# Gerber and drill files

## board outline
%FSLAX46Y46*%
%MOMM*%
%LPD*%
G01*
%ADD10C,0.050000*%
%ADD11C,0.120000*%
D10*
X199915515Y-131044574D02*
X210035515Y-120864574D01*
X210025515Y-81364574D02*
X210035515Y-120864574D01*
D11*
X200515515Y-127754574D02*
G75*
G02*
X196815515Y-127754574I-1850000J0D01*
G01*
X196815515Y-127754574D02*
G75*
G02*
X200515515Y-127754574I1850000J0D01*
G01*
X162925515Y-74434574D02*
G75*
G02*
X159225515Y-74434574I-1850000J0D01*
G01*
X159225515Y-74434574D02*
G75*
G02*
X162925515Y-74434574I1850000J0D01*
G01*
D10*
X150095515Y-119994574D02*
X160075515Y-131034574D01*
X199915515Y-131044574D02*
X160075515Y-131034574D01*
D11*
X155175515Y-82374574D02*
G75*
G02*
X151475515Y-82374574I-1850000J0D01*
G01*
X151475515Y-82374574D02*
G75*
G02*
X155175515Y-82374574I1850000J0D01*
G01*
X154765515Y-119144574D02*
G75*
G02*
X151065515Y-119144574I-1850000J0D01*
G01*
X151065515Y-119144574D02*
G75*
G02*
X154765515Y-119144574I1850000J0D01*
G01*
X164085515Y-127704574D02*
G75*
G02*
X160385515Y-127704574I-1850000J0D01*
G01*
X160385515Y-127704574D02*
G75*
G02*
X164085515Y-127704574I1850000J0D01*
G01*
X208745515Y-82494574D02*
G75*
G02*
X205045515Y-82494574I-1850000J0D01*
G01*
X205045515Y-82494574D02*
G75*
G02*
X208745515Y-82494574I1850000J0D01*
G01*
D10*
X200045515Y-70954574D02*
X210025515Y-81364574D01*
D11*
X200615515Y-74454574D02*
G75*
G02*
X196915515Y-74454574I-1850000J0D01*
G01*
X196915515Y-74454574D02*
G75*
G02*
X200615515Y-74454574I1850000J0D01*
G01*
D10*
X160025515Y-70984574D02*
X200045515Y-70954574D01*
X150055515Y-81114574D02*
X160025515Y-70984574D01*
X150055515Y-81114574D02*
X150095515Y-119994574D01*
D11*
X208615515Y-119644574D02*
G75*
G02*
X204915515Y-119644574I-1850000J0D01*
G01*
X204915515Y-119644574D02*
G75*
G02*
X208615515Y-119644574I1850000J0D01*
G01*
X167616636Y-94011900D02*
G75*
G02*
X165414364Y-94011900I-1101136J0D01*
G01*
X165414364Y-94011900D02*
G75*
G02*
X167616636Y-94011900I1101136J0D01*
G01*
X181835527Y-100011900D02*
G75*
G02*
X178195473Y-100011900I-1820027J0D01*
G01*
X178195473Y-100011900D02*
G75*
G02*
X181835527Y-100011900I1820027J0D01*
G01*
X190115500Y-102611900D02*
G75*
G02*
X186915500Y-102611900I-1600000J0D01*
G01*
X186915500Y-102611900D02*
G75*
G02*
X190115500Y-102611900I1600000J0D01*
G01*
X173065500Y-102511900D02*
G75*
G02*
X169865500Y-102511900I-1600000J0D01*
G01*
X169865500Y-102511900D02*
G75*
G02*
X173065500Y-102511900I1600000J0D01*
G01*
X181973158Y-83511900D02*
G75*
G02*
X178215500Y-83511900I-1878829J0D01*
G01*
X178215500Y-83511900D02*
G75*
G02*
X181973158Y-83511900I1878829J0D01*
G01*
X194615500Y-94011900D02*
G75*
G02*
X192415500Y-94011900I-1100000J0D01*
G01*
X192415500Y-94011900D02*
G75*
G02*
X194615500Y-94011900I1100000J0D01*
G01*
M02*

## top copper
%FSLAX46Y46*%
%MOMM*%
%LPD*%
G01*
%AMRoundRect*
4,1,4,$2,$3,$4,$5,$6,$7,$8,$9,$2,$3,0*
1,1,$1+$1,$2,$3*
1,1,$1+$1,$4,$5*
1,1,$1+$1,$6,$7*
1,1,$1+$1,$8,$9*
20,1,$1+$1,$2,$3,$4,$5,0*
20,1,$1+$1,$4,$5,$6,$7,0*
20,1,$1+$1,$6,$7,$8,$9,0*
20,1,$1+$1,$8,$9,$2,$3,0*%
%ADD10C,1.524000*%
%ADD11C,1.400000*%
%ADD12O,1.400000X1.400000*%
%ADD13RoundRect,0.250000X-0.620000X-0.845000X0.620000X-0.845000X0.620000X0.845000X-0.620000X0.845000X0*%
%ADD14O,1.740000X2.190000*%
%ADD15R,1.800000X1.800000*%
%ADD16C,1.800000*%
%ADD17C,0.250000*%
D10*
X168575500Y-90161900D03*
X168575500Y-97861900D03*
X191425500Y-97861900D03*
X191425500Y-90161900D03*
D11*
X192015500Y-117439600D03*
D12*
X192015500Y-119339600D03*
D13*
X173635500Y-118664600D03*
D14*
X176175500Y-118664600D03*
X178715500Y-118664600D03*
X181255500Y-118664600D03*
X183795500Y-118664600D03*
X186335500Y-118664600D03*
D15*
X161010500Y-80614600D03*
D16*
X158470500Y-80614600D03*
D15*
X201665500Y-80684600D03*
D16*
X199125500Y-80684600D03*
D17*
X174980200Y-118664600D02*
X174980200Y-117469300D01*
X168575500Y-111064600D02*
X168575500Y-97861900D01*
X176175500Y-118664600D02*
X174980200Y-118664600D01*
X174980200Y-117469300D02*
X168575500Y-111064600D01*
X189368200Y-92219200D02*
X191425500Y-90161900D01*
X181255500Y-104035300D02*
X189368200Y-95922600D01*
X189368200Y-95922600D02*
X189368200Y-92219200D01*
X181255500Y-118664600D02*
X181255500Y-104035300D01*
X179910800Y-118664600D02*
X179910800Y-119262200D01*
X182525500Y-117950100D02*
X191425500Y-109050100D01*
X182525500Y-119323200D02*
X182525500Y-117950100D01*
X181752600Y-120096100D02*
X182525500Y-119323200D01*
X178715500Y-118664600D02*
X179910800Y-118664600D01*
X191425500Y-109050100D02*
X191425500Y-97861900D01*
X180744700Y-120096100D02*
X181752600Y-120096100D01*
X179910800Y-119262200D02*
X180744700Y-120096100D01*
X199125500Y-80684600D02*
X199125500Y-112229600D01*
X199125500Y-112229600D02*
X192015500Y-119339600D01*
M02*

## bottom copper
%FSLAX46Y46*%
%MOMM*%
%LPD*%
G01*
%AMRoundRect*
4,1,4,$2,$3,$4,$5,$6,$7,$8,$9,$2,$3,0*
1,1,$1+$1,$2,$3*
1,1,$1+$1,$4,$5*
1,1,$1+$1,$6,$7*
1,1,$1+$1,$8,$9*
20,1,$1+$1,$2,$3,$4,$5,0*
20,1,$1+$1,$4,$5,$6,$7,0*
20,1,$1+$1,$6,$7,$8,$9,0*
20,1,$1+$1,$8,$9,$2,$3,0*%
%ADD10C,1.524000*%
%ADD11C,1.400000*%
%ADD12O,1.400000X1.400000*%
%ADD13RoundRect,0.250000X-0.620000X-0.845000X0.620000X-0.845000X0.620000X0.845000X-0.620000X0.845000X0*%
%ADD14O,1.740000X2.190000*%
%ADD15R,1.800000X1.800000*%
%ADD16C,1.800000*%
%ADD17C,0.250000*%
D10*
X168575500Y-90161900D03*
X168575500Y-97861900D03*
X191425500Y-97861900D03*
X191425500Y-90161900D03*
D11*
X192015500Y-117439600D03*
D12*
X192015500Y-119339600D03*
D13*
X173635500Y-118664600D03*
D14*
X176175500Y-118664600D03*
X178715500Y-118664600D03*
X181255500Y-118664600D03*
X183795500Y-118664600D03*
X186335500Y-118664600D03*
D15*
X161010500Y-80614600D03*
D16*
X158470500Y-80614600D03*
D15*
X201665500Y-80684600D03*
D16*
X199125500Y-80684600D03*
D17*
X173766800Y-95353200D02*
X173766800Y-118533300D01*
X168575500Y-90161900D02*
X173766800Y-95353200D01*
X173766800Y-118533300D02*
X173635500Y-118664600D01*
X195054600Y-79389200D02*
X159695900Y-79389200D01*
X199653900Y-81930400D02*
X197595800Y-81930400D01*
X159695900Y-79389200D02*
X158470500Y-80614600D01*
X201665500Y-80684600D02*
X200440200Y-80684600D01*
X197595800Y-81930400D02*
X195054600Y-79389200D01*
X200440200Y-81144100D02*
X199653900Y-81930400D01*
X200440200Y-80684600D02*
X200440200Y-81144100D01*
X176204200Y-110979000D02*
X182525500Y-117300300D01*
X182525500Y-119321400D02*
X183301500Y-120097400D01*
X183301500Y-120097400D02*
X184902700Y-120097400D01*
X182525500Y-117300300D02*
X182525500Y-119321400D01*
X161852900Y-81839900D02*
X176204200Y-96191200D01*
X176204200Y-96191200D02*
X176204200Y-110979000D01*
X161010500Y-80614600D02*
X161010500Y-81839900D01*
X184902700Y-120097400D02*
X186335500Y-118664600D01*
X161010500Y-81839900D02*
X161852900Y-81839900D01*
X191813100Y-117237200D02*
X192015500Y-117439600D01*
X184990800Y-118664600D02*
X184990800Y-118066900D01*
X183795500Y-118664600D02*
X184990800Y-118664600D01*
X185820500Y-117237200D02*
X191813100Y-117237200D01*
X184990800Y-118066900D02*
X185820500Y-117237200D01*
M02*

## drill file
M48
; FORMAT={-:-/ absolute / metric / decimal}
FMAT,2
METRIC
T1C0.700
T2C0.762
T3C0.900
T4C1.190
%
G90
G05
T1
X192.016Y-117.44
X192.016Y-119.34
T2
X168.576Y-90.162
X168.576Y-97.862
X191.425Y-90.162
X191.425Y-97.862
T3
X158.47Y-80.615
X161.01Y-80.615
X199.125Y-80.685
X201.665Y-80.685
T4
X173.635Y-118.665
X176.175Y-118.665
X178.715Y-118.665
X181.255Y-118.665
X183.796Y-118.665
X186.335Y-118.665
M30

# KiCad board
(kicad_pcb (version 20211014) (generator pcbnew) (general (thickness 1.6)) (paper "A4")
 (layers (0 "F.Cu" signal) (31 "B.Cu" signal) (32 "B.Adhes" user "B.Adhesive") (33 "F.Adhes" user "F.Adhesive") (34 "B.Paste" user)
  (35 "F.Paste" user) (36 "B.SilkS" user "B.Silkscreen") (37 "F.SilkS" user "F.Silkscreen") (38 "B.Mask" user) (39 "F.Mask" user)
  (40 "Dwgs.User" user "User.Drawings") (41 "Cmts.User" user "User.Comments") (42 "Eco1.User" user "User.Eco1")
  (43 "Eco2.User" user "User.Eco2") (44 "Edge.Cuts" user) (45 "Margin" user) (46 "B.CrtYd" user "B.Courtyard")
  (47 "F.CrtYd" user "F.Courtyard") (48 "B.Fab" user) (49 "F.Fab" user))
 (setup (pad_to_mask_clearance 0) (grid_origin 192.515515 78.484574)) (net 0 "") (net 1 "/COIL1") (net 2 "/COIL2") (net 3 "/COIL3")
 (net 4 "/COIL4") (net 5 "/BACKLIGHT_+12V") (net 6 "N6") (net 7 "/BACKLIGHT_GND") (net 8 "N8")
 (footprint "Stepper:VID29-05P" (layer "F.Cu") (at 180.0155 94.0119)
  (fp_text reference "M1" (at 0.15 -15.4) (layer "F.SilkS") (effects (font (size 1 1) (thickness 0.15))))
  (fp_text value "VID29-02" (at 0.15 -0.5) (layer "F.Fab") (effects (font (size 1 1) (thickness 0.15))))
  (fp_circle (center -13.5 0) (end -12.65 0.7) (layer "Edge.Cuts") (width 0.12) (fill none))
  (fp_circle (center 0 6) (end 1.45 7.1) (layer "Edge.Cuts") (width 0.12) (fill none))
  (fp_circle (center 8.5 8.6) (end 10.1 8.6) (layer "Edge.Cuts") (width 0.12) (fill none))
  (fp_circle (center -8.55 8.5) (end -6.95 8.5) (layer "Edge.Cuts") (width 0.12) (fill none))
  (fp_circle (center 0.078829 -10.5) (end 1.778829 -9.7) (layer "Edge.Cuts") (width 0.12) (fill none))
  (fp_circle (center 13.5 0) (end 14.6 0) (layer "Edge.Cuts") (width 0.12) (fill none))
  (pad "1" thru_hole circle (at -11.44 -3.85) (size 1.524 1.524) (drill 0.762) (layers *.Cu *.Mask) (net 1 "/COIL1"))
  (pad "2" thru_hole circle (at -11.44 3.85) (size 1.524 1.524) (drill 0.762) (layers *.Cu *.Mask) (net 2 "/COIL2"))
  (pad "3" thru_hole circle (at 11.41 3.85) (size 1.524 1.524) (drill 0.762) (layers *.Cu *.Mask) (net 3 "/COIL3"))
  (pad "4" thru_hole circle (at 11.41 -3.85) (size 1.524 1.524) (drill 0.762) (layers *.Cu *.Mask) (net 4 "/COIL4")))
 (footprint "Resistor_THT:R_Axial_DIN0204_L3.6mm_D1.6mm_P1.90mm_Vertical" (layer "F.Cu") (at 192.0155 117.4396 -90)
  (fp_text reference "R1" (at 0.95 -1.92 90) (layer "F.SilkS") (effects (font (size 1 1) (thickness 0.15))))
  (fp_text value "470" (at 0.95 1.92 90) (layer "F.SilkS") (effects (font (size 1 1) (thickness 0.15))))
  (pad "1" thru_hole circle (at 0 0 270) (size 1.4 1.4) (drill 0.7) (layers *.Cu *.Mask) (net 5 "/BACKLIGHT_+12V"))
  (pad "2" thru_hole oval (at 1.9 0 270) (size 1.4 1.4) (drill 0.7) (layers *.Cu *.Mask) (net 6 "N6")))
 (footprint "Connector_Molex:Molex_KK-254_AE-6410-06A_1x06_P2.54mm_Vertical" (layer "F.Cu") (at 173.6355 118.6646)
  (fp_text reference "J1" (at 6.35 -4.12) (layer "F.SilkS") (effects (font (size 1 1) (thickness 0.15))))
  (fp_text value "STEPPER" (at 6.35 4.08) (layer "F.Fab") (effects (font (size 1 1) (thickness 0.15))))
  (pad "1" thru_hole roundrect (at 0 0) (size 1.74 2.19) (drill 1.19) (layers *.Cu *.Mask) (roundrect_rratio 0.1436781609) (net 1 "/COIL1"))
  (pad "2" thru_hole oval (at 2.54 0) (size 1.74 2.19) (drill 1.19) (layers *.Cu *.Mask) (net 2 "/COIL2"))
  (pad "3" thru_hole oval (at 5.08 0) (size 1.74 2.19) (drill 1.19) (layers *.Cu *.Mask) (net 3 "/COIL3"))
  (pad "4" thru_hole oval (at 7.62 0) (size 1.74 2.19) (drill 1.19) (layers *.Cu *.Mask) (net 4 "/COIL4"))
  (pad "5" thru_hole oval (at 10.16 0) (size 1.74 2.19) (drill 1.19) (layers *.Cu *.Mask) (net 5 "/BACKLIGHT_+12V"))
  (pad "6" thru_hole oval (at 12.7 0) (size 1.74 2.19) (drill 1.19) (layers *.Cu *.Mask) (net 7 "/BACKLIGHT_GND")))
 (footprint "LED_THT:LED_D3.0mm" (layer "B.Cu") (at 161.0105 80.6146 180)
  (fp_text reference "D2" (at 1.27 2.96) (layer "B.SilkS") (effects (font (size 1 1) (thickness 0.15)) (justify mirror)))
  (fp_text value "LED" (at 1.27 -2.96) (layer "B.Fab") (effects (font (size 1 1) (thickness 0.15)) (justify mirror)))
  (pad "1" thru_hole rect (at 0 0 180) (size 1.8 1.8) (drill 0.9) (layers *.Cu *.Mask) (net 7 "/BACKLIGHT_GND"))
  (pad "2" thru_hole circle (at 2.54 0 180) (size 1.8 1.8) (drill 0.9) (layers *.Cu *.Mask) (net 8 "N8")))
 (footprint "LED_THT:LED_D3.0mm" (layer "B.Cu") (at 201.6655 80.6846 180)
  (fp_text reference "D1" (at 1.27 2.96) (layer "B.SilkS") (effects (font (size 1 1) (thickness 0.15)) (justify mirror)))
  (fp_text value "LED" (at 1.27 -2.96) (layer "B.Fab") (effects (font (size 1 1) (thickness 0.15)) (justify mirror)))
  (pad "1" thru_hole rect (at 0 0 180) (size 1.8 1.8) (drill 0.9) (layers *.Cu *.Mask) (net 8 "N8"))
  (pad "2" thru_hole circle (at 2.54 0 180) (size 1.8 1.8) (drill 0.9) (layers *.Cu *.Mask) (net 6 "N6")))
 (gr_line (start 199.915515 131.044574) (end 210.035515 120.864574) (layer "Edge.Cuts") (width 0.05))
 (gr_line (start 210.025515 81.364574) (end 210.035515 120.864574) (layer "Edge.Cuts") (width 0.05))
 (gr_circle (center 198.665515 127.754574) (end 200.515515 127.754574) (layer "Edge.Cuts") (width 0.12) (fill none))
 (gr_circle (center 161.075515 74.434574) (end 162.925515 74.434574) (layer "Edge.Cuts") (width 0.12) (fill none))
 (gr_line (start 150.095515 119.994574) (end 160.075515 131.034574) (layer "Edge.Cuts") (width 0.05))
 (gr_line (start 199.915515 131.044574) (end 160.075515 131.034574) (layer "Edge.Cuts") (width 0.05))
 (gr_circle (center 153.325515 82.374574) (end 155.175515 82.374574) (layer "Edge.Cuts") (width 0.12) (fill none))
 (gr_circle (center 152.915515 119.144574) (end 154.765515 119.144574) (layer "Edge.Cuts") (width 0.12) (fill none))
 (gr_circle (center 162.235515 127.704574) (end 164.085515 127.704574) (layer "Edge.Cuts") (width 0.12) (fill none))
 (gr_circle (center 206.895515 82.494574) (end 208.745515 82.494574) (layer "Edge.Cuts") (width 0.12) (fill none))
 (gr_line (start 200.045515 70.954574) (end 210.025515 81.364574) (layer "Edge.Cuts") (width 0.05))
 (gr_circle (center 198.765515 74.454574) (end 200.615515 74.454574) (layer "Edge.Cuts") (width 0.12) (fill none))
 (gr_line (start 160.025515 70.984574) (end 200.045515 70.954574) (layer "Edge.Cuts") (width 0.05))
 (gr_line (start 150.055515 81.114574) (end 160.025515 70.984574) (layer "Edge.Cuts") (width 0.05))
 (gr_line (start 150.055515 81.114574) (end 150.095515 119.994574) (layer "Edge.Cuts") (width 0.05))
 (gr_circle (center 206.765515 119.644574) (end 208.615515 119.644574) (layer "Edge.Cuts") (width 0.12) (fill none))
 (segment (start 174.9802 118.6646) (end 174.9802 117.4693) (width 0.25) (layer "F.Cu") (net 2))
 (segment (start 168.5755 111.0646) (end 168.5755 97.8619) (width 0.25) (layer "F.Cu") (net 2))
 (segment (start 176.1755 118.6646) (end 174.9802 118.6646) (width 0.25) (layer "F.Cu") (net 2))
 (segment (start 174.9802 117.4693) (end 168.5755 111.0646) (width 0.25) (layer "F.Cu") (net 2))
 (segment (start 173.7668 95.3532) (end 173.7668 118.5333) (width 0.25) (layer "B.Cu") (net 1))
 (segment (start 168.5755 90.1619) (end 173.7668 95.3532) (width 0.25) (layer "B.Cu") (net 1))
 (segment (start 173.7668 118.5333) (end 173.6355 118.6646) (width 0.25) (layer "B.Cu") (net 1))
 (segment (start 189.3682 92.2192) (end 191.4255 90.1619) (width 0.25) (layer "F.Cu") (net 4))
 (segment (start 181.2555 104.0353) (end 189.3682 95.9226) (width 0.25) (layer "F.Cu") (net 4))
 (segment (start 189.3682 95.9226) (end 189.3682 92.2192) (width 0.25) (layer "F.Cu") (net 4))
 (segment (start 181.2555 118.6646) (end 181.2555 104.0353) (width 0.25) (layer "F.Cu") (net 4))
 (segment (start 179.9108 118.6646) (end 179.9108 119.2622) (width 0.25) (layer "F.Cu") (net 3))
 (segment (start 182.5255 117.9501) (end 191.4255 109.0501) (width 0.25) (layer "F.Cu") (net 3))
 (segment (start 182.5255 119.3232) (end 182.5255 117.9501) (width 0.25) (layer "F.Cu") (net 3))
 (segment (start 181.7526 120.0961) (end 182.5255 119.3232) (width 0.25) (layer "F.Cu") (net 3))
 (segment (start 178.7155 118.6646) (end 179.9108 118.6646) (width 0.25) (layer "F.Cu") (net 3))
 (segment (start 191.4255 109.0501) (end 191.4255 97.8619) (width 0.25) (layer "F.Cu") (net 3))
 (segment (start 180.7447 120.0961) (end 181.7526 120.0961) (width 0.25) (layer "F.Cu") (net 3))
 (segment (start 179.9108 119.2622) (end 180.7447 120.0961) (width 0.25) (layer "F.Cu") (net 3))
 (segment (start 195.0546 79.3892) (end 159.6959 79.3892) (width 0.25) (layer "B.Cu") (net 8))
 (segment (start 199.6539 81.9304) (end 197.5958 81.9304) (width 0.25) (layer "B.Cu") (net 8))
 (segment (start 159.6959 79.3892) (end 158.4705 80.6146) (width 0.25) (layer "B.Cu") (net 8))
 (segment (start 201.6655 80.6846) (end 200.4402 80.6846) (width 0.25) (layer "B.Cu") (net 8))
 (segment (start 197.5958 81.9304) (end 195.0546 79.3892) (width 0.25) (layer "B.Cu") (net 8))
 (segment (start 200.4402 81.1441) (end 199.6539 81.9304) (width 0.25) (layer "B.Cu") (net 8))
 (segment (start 200.4402 80.6846) (end 200.4402 81.1441) (width 0.25) (layer "B.Cu") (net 8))
 (segment (start 199.1255 80.6846) (end 199.1255 112.2296) (width 0.25) (layer "F.Cu") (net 6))
 (segment (start 199.1255 112.2296) (end 192.0155 119.3396) (width 0.25) (layer "F.Cu") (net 6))
 (segment (start 176.2042 110.979) (end 182.5255 117.3003) (width 0.25) (layer "B.Cu") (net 7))
 (segment (start 182.5255 119.3214) (end 183.3015 120.0974) (width 0.25) (layer "B.Cu") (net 7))
 (segment (start 183.3015 120.0974) (end 184.9027 120.0974) (width 0.25) (layer "B.Cu") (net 7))
 (segment (start 182.5255 117.3003) (end 182.5255 119.3214) (width 0.25) (layer "B.Cu") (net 7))
 (segment (start 161.8529 81.8399) (end 176.2042 96.1912) (width 0.25) (layer "B.Cu") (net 7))
 (segment (start 176.2042 96.1912) (end 176.2042 110.979) (width 0.25) (layer "B.Cu") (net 7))
 (segment (start 161.0105 80.6146) (end 161.0105 81.8399) (width 0.25) (layer "B.Cu") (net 7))
 (segment (start 184.9027 120.0974) (end 186.3355 118.6646) (width 0.25) (layer "B.Cu") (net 7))
 (segment (start 161.0105 81.8399) (end 161.8529 81.8399) (width 0.25) (layer "B.Cu") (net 7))
 (segment (start 191.8131 117.2372) (end 192.0155 117.4396) (width 0.25) (layer "B.Cu") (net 5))
 (segment (start 184.9908 118.6646) (end 184.9908 118.0669) (width 0.25) (layer "B.Cu") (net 5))
 (segment (start 183.7955 118.6646) (end 184.9908 118.6646) (width 0.25) (layer "B.Cu") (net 5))
 (segment (start 185.8205 117.2372) (end 191.8131 117.2372) (width 0.25) (layer "B.Cu") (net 5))
 (segment (start 184.9908 118.0669) (end 185.8205 117.2372) (width 0.25) (layer "B.Cu") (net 5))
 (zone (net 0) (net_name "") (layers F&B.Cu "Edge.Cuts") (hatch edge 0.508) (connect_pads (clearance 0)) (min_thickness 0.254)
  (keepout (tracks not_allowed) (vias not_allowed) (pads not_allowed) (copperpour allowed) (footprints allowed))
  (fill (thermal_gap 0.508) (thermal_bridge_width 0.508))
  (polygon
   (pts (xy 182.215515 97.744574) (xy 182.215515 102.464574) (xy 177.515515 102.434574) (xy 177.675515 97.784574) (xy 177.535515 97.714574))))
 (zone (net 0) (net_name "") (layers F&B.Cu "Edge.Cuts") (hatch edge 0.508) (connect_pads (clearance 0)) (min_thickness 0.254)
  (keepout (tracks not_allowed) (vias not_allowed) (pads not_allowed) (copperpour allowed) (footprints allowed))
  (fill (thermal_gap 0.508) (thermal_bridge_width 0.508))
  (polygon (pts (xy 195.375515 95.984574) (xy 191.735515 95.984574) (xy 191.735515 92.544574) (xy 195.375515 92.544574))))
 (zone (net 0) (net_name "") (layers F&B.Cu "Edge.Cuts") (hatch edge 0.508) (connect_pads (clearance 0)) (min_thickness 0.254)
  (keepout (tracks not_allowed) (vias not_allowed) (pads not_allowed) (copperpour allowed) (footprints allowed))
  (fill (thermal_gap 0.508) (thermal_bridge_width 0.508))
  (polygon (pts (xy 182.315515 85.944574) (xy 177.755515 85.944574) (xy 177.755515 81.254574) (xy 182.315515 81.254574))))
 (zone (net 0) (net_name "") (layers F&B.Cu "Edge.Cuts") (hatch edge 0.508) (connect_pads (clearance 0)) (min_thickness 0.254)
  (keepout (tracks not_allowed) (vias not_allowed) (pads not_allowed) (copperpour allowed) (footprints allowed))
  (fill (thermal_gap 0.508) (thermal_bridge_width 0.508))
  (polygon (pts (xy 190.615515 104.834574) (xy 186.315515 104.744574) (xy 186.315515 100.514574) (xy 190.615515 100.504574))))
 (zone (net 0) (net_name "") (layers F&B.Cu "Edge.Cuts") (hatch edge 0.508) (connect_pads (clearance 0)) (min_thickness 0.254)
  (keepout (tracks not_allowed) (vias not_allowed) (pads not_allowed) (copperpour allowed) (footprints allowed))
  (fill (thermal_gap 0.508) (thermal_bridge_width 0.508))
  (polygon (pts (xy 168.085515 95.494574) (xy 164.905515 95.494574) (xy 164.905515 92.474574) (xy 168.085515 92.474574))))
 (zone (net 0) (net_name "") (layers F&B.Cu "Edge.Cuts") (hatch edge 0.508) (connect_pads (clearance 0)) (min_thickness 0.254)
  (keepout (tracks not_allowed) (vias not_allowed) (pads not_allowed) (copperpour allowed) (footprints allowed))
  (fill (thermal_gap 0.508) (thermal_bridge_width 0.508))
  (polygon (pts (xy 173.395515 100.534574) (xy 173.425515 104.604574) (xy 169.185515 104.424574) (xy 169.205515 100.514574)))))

